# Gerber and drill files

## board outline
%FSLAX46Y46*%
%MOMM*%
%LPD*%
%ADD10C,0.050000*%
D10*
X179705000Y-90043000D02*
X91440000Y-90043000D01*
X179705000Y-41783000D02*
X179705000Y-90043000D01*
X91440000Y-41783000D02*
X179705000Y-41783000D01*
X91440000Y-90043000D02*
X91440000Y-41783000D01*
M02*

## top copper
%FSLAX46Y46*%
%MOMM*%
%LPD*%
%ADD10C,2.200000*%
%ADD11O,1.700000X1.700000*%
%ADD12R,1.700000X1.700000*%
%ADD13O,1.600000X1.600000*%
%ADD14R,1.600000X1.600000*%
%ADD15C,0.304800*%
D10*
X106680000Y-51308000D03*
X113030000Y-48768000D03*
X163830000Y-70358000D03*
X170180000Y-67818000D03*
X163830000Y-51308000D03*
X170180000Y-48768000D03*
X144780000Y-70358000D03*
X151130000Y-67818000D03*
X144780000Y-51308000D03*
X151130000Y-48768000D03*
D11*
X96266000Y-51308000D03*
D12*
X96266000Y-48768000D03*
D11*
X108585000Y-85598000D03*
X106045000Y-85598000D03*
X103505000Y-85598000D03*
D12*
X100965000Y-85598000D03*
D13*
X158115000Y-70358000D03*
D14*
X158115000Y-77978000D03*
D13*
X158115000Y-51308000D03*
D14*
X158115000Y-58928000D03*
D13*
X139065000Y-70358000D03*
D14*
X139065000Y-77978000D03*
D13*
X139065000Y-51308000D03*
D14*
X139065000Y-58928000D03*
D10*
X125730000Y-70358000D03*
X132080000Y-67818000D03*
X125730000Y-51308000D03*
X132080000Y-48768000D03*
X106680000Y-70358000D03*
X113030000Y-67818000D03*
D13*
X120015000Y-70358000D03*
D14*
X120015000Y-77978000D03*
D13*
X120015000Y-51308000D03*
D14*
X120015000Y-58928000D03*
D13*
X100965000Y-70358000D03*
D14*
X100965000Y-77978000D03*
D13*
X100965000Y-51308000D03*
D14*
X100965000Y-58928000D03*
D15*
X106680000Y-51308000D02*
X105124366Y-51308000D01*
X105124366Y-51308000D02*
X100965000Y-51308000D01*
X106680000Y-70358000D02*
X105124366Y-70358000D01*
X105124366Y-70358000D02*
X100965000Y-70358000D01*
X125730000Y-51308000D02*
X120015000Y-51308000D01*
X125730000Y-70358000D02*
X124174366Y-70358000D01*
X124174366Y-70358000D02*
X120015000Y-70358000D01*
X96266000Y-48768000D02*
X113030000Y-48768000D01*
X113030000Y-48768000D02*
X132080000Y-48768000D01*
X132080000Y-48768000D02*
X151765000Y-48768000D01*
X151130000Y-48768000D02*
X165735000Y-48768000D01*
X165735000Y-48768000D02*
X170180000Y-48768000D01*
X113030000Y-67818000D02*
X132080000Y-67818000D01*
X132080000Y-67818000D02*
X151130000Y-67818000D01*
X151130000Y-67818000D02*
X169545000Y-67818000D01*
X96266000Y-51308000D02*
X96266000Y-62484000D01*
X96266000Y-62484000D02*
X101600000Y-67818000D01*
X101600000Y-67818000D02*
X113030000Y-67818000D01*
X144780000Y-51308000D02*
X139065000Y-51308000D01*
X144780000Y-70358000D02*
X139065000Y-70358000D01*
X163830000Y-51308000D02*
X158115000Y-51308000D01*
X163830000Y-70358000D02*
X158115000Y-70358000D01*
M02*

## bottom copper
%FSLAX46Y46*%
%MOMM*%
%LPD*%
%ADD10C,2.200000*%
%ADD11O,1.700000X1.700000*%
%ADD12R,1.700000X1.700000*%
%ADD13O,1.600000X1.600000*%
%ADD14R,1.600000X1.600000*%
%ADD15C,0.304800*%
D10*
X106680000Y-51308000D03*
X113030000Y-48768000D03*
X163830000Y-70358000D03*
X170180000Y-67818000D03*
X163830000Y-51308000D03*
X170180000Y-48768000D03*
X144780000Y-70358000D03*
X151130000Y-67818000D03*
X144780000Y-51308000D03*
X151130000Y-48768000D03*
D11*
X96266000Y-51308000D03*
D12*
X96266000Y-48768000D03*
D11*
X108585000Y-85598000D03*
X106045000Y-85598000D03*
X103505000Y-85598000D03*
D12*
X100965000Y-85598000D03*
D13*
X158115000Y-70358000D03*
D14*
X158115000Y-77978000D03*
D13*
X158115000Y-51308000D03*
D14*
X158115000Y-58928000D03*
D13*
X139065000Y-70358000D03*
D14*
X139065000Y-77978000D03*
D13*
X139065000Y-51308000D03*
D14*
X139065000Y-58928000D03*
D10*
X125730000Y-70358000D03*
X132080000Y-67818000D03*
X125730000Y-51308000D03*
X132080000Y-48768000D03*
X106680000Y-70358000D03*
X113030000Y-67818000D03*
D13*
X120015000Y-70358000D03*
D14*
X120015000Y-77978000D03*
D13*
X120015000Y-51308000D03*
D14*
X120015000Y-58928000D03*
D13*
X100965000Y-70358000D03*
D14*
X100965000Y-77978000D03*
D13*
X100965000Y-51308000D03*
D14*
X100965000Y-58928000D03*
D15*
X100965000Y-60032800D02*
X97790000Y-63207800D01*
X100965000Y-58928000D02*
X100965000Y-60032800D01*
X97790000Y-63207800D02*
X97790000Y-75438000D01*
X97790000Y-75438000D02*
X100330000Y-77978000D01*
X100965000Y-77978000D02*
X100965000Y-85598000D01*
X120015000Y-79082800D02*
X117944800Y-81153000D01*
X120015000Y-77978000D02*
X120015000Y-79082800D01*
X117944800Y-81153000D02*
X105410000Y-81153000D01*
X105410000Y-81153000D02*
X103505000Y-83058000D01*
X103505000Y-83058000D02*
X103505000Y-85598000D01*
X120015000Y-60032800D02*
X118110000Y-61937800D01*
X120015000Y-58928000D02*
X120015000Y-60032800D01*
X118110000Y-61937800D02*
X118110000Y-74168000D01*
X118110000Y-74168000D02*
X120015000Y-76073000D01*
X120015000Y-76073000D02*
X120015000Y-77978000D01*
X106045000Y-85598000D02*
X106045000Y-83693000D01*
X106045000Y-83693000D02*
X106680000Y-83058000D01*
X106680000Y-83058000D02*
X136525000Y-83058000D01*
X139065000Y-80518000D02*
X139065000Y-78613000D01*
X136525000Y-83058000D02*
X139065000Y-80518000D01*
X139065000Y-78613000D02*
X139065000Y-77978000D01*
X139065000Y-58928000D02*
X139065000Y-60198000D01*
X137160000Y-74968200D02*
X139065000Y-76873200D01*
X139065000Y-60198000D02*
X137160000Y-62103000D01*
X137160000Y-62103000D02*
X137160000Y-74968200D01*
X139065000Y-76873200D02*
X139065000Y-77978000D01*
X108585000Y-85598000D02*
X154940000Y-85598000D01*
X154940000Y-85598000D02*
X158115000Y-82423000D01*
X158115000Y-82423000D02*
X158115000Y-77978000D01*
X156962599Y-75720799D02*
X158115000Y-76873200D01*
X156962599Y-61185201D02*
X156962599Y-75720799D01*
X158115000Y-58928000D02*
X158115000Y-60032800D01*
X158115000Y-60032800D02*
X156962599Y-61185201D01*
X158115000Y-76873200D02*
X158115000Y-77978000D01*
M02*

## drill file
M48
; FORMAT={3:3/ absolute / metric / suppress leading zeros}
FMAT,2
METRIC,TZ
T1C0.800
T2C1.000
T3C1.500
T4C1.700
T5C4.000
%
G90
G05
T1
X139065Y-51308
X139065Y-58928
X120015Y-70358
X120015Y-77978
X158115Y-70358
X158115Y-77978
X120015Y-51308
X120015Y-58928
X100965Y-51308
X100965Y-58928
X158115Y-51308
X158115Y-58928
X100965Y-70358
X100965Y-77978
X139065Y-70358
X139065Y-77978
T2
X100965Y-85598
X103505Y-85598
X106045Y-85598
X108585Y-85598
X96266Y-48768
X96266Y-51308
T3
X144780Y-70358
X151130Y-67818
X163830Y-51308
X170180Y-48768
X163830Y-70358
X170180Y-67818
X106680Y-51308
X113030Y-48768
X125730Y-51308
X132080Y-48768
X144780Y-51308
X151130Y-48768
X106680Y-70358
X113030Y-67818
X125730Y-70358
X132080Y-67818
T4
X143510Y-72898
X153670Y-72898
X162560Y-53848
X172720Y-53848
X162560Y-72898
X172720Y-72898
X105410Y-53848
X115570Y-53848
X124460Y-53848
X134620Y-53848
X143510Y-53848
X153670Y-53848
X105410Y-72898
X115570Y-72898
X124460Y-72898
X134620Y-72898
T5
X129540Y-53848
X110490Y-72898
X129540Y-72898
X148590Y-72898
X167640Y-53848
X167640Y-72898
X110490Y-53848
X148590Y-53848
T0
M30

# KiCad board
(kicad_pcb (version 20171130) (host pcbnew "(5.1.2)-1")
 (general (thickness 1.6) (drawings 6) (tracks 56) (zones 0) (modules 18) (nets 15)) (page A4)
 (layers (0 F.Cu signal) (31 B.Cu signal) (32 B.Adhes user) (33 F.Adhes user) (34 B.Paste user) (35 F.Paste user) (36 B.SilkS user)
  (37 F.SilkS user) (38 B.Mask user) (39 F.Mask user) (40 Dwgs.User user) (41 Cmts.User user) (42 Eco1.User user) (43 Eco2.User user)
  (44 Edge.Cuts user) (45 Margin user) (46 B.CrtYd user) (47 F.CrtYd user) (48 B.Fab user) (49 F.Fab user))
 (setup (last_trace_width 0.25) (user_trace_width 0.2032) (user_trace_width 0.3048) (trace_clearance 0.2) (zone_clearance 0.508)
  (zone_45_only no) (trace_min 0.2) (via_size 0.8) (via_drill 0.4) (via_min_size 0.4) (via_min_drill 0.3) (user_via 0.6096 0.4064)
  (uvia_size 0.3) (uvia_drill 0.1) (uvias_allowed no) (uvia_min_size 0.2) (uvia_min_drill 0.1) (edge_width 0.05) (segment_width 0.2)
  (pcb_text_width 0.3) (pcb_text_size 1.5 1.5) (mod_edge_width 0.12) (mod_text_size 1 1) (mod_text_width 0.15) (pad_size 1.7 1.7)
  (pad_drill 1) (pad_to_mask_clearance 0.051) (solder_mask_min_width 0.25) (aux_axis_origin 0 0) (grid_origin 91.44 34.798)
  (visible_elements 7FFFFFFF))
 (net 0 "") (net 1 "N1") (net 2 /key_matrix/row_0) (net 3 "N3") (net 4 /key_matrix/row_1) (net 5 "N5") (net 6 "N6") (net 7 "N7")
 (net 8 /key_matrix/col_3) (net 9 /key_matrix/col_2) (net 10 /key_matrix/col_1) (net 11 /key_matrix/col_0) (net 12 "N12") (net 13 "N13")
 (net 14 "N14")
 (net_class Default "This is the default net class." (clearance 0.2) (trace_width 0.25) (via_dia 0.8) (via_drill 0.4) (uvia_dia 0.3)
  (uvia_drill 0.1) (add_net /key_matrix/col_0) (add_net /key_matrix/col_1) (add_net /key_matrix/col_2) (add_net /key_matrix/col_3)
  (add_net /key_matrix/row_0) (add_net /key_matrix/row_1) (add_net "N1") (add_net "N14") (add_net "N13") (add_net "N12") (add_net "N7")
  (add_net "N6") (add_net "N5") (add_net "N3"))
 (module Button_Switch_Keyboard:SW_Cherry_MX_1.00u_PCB (layer F.Cu) (at 113.03 48.768)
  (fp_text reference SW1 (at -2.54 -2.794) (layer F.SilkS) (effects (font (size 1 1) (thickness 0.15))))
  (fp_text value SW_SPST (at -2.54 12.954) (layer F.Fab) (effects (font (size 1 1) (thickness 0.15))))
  (pad "" np_thru_hole circle (at 2.54 5.08) (size 1.7 1.7) (drill 1.7) (layers *.Cu *.Mask))
  (pad "" np_thru_hole circle (at -7.62 5.08) (size 1.7 1.7) (drill 1.7) (layers *.Cu *.Mask))
  (pad "" np_thru_hole circle (at -2.54 5.08) (size 4 4) (drill 4) (layers *.Cu *.Mask))
  (pad 2 thru_hole circle (at -6.35 2.54) (size 2.2 2.2) (drill 1.5) (layers *.Cu *.Mask) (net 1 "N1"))
  (pad 1 thru_hole circle (at 0 0) (size 2.2 2.2) (drill 1.5) (layers *.Cu *.Mask) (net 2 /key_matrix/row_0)))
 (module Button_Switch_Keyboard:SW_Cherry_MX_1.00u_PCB (layer F.Cu) (at 170.18 67.818)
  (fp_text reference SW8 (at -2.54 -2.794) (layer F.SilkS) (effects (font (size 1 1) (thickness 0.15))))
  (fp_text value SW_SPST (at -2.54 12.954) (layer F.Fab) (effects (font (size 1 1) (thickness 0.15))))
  (pad "" np_thru_hole circle (at 2.54 5.08) (size 1.7 1.7) (drill 1.7) (layers *.Cu *.Mask))
  (pad "" np_thru_hole circle (at -7.62 5.08) (size 1.7 1.7) (drill 1.7) (layers *.Cu *.Mask))
  (pad "" np_thru_hole circle (at -2.54 5.08) (size 4 4) (drill 4) (layers *.Cu *.Mask))
  (pad 2 thru_hole circle (at -6.35 2.54) (size 2.2 2.2) (drill 1.5) (layers *.Cu *.Mask) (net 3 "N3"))
  (pad 1 thru_hole circle (at 0 0) (size 2.2 2.2) (drill 1.5) (layers *.Cu *.Mask) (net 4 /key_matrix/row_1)))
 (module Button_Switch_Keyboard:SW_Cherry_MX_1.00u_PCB (layer F.Cu) (at 170.18 48.768)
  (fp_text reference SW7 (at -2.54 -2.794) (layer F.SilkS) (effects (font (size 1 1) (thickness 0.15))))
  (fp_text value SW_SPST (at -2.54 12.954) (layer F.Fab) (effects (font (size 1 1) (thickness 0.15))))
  (pad "" np_thru_hole circle (at 2.54 5.08) (size 1.7 1.7) (drill 1.7) (layers *.Cu *.Mask))
  (pad "" np_thru_hole circle (at -7.62 5.08) (size 1.7 1.7) (drill 1.7) (layers *.Cu *.Mask))
  (pad "" np_thru_hole circle (at -2.54 5.08) (size 4 4) (drill 4) (layers *.Cu *.Mask))
  (pad 2 thru_hole circle (at -6.35 2.54) (size 2.2 2.2) (drill 1.5) (layers *.Cu *.Mask) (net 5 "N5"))
  (pad 1 thru_hole circle (at 0 0) (size 2.2 2.2) (drill 1.5) (layers *.Cu *.Mask) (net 2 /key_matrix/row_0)))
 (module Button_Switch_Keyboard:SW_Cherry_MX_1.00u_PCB (layer F.Cu) (at 151.13 67.818)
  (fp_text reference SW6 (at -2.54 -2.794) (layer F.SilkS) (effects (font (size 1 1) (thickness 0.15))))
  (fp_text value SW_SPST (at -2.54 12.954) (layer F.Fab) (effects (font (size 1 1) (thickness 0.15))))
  (pad "" np_thru_hole circle (at 2.54 5.08) (size 1.7 1.7) (drill 1.7) (layers *.Cu *.Mask))
  (pad "" np_thru_hole circle (at -7.62 5.08) (size 1.7 1.7) (drill 1.7) (layers *.Cu *.Mask))
  (pad "" np_thru_hole circle (at -2.54 5.08) (size 4 4) (drill 4) (layers *.Cu *.Mask))
  (pad 2 thru_hole circle (at -6.35 2.54) (size 2.2 2.2) (drill 1.5) (layers *.Cu *.Mask) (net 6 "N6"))
  (pad 1 thru_hole circle (at 0 0) (size 2.2 2.2) (drill 1.5) (layers *.Cu *.Mask) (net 4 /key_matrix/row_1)))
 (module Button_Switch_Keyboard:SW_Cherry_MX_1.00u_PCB (layer F.Cu) (at 151.13 48.768)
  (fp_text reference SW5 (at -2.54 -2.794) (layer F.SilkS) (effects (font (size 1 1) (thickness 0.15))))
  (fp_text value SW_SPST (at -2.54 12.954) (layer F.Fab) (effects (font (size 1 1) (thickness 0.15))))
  (pad "" np_thru_hole circle (at 2.54 5.08) (size 1.7 1.7) (drill 1.7) (layers *.Cu *.Mask))
  (pad "" np_thru_hole circle (at -7.62 5.08) (size 1.7 1.7) (drill 1.7) (layers *.Cu *.Mask))
  (pad "" np_thru_hole circle (at -2.54 5.08) (size 4 4) (drill 4) (layers *.Cu *.Mask))
  (pad 2 thru_hole circle (at -6.35 2.54) (size 2.2 2.2) (drill 1.5) (layers *.Cu *.Mask) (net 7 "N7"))
  (pad 1 thru_hole circle (at 0 0) (size 2.2 2.2) (drill 1.5) (layers *.Cu *.Mask) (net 2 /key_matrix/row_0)))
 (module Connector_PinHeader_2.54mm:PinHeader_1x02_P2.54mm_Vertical (layer F.Cu) (at 96.266 48.768)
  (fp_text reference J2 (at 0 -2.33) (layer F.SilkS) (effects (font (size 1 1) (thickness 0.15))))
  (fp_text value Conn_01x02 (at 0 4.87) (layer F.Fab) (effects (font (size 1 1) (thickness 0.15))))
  (pad 2 thru_hole oval (at 0 2.54) (size 1.7 1.7) (drill 1) (layers *.Cu *.Mask) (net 4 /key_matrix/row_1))
  (pad 1 thru_hole rect (at 0 0) (size 1.7 1.7) (drill 1) (layers *.Cu *.Mask) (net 2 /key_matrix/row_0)))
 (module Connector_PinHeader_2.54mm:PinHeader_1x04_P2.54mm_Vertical (layer F.Cu) (at 100.965 85.598 90)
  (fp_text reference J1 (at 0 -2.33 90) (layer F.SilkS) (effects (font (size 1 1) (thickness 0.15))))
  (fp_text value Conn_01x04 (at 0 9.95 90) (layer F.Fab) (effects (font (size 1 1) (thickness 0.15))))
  (pad 4 thru_hole oval (at 0 7.62 90) (size 1.7 1.7) (drill 1) (layers *.Cu *.Mask) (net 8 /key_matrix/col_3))
  (pad 3 thru_hole oval (at 0 5.08 90) (size 1.7 1.7) (drill 1) (layers *.Cu *.Mask) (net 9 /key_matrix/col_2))
  (pad 2 thru_hole oval (at 0 2.54 90) (size 1.7 1.7) (drill 1) (layers *.Cu *.Mask) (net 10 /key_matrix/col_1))
  (pad 1 thru_hole rect (at 0 0 90) (size 1.7 1.7) (drill 1) (layers *.Cu *.Mask) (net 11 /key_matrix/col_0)))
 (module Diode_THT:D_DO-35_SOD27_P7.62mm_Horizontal (layer F.Cu) (at 158.115 77.978 90)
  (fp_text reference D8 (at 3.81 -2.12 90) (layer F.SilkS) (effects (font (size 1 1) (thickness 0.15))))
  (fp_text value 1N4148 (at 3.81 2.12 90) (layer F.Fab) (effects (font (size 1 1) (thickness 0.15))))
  (pad 2 thru_hole oval (at 7.62 0 90) (size 1.6 1.6) (drill 0.8) (layers *.Cu *.Mask) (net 3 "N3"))
  (pad 1 thru_hole rect (at 0 0 90) (size 1.6 1.6) (drill 0.8) (layers *.Cu *.Mask) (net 8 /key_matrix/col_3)))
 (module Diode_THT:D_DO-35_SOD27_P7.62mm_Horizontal (layer F.Cu) (at 158.115 58.928 90)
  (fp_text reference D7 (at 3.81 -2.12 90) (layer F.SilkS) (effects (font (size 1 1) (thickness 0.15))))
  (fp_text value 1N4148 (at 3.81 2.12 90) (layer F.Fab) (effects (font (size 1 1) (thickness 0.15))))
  (pad 2 thru_hole oval (at 7.62 0 90) (size 1.6 1.6) (drill 0.8) (layers *.Cu *.Mask) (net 5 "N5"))
  (pad 1 thru_hole rect (at 0 0 90) (size 1.6 1.6) (drill 0.8) (layers *.Cu *.Mask) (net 8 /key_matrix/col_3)))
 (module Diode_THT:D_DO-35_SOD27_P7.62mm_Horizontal (layer F.Cu) (at 139.065 77.978 90)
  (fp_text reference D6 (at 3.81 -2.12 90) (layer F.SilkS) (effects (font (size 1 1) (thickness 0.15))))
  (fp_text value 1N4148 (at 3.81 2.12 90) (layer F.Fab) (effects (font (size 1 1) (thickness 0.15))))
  (pad 2 thru_hole oval (at 7.62 0 90) (size 1.6 1.6) (drill 0.8) (layers *.Cu *.Mask) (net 6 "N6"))
  (pad 1 thru_hole rect (at 0 0 90) (size 1.6 1.6) (drill 0.8) (layers *.Cu *.Mask) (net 9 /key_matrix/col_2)))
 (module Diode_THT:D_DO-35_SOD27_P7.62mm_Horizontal (layer F.Cu) (at 139.065 58.928 90)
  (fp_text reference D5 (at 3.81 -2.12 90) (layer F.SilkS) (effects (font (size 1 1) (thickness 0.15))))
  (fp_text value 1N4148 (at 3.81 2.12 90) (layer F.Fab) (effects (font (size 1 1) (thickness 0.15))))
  (pad 2 thru_hole oval (at 7.62 0 90) (size 1.6 1.6) (drill 0.8) (layers *.Cu *.Mask) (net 7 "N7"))
  (pad 1 thru_hole rect (at 0 0 90) (size 1.6 1.6) (drill 0.8) (layers *.Cu *.Mask) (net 9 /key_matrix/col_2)))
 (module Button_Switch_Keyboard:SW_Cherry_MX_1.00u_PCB (layer F.Cu) (at 132.08 67.818)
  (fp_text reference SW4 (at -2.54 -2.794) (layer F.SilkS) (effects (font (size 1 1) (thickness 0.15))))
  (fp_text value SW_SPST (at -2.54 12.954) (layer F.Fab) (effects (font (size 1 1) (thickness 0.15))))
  (pad "" np_thru_hole circle (at 2.54 5.08) (size 1.7 1.7) (drill 1.7) (layers *.Cu *.Mask))
  (pad "" np_thru_hole circle (at -7.62 5.08) (size 1.7 1.7) (drill 1.7) (layers *.Cu *.Mask))
  (pad "" np_thru_hole circle (at -2.54 5.08) (size 4 4) (drill 4) (layers *.Cu *.Mask))
  (pad 2 thru_hole circle (at -6.35 2.54) (size 2.2 2.2) (drill 1.5) (layers *.Cu *.Mask) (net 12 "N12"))
  (pad 1 thru_hole circle (at 0 0) (size 2.2 2.2) (drill 1.5) (layers *.Cu *.Mask) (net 4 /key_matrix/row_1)))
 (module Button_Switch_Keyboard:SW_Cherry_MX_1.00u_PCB (layer F.Cu) (at 132.08 48.768)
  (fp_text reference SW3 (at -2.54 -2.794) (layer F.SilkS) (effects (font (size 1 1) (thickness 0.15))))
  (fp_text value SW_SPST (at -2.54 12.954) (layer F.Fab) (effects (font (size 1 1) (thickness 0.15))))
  (pad "" np_thru_hole circle (at 2.54 5.08) (size 1.7 1.7) (drill 1.7) (layers *.Cu *.Mask))
  (pad "" np_thru_hole circle (at -7.62 5.08) (size 1.7 1.7) (drill 1.7) (layers *.Cu *.Mask))
  (pad "" np_thru_hole circle (at -2.54 5.08) (size 4 4) (drill 4) (layers *.Cu *.Mask))
  (pad 2 thru_hole circle (at -6.35 2.54) (size 2.2 2.2) (drill 1.5) (layers *.Cu *.Mask) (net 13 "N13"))
  (pad 1 thru_hole circle (at 0 0) (size 2.2 2.2) (drill 1.5) (layers *.Cu *.Mask) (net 2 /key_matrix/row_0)))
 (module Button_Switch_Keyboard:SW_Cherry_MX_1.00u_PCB (layer F.Cu) (at 113.03 67.818)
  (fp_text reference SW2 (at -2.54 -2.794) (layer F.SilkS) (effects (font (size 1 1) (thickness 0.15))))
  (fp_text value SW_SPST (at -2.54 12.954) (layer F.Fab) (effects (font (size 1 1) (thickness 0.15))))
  (pad "" np_thru_hole circle (at 2.54 5.08) (size 1.7 1.7) (drill 1.7) (layers *.Cu *.Mask))
  (pad "" np_thru_hole circle (at -7.62 5.08) (size 1.7 1.7) (drill 1.7) (layers *.Cu *.Mask))
  (pad "" np_thru_hole circle (at -2.54 5.08) (size 4 4) (drill 4) (layers *.Cu *.Mask))
  (pad 2 thru_hole circle (at -6.35 2.54) (size 2.2 2.2) (drill 1.5) (layers *.Cu *.Mask) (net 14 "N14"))
  (pad 1 thru_hole circle (at 0 0) (size 2.2 2.2) (drill 1.5) (layers *.Cu *.Mask) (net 4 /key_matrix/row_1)))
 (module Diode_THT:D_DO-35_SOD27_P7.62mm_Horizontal (layer F.Cu) (at 120.015 77.978 90)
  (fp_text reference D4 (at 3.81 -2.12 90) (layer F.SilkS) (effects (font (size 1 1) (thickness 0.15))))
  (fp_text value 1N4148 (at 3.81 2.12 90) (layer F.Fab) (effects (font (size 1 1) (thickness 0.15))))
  (pad 2 thru_hole oval (at 7.62 0 90) (size 1.6 1.6) (drill 0.8) (layers *.Cu *.Mask) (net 12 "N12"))
  (pad 1 thru_hole rect (at 0 0 90) (size 1.6 1.6) (drill 0.8) (layers *.Cu *.Mask) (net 10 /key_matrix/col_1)))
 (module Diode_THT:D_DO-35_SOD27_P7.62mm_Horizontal (layer F.Cu) (at 120.015 58.928 90)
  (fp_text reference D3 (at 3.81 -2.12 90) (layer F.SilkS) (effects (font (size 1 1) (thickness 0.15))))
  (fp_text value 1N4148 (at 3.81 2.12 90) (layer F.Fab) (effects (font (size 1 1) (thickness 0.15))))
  (pad 2 thru_hole oval (at 7.62 0 90) (size 1.6 1.6) (drill 0.8) (layers *.Cu *.Mask) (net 13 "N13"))
  (pad 1 thru_hole rect (at 0 0 90) (size 1.6 1.6) (drill 0.8) (layers *.Cu *.Mask) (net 10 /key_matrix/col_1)))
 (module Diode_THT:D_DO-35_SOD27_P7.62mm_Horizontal (layer F.Cu) (at 100.965 77.978 90)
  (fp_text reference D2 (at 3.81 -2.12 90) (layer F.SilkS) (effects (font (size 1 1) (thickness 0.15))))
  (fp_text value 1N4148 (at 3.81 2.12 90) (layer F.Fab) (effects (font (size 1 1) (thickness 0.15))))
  (pad 2 thru_hole oval (at 7.62 0 90) (size 1.6 1.6) (drill 0.8) (layers *.Cu *.Mask) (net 14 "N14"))
  (pad 1 thru_hole rect (at 0 0 90) (size 1.6 1.6) (drill 0.8) (layers *.Cu *.Mask) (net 11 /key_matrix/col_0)))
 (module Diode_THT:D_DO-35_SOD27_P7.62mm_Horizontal (layer F.Cu) (at 100.965 58.928 90)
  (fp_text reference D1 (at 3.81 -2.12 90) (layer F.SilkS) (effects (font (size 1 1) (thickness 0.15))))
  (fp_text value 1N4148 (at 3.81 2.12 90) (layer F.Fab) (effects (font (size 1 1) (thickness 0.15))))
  (pad 2 thru_hole oval (at 7.62 0 90) (size 1.6 1.6) (drill 0.8) (layers *.Cu *.Mask) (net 1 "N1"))
  (pad 1 thru_hole rect (at 0 0 90) (size 1.6 1.6) (drill 0.8) (layers *.Cu *.Mask) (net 11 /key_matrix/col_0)))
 (gr_line (start 179.705 90.043) (end 91.44 90.043) (layer Edge.Cuts) (width 0.05))
 (gr_line (start 179.705 41.783) (end 179.705 90.043) (layer Edge.Cuts) (width 0.05))
 (gr_line (start 91.44 41.783) (end 179.705 41.783) (layer Edge.Cuts) (width 0.05))
 (gr_line (start 91.44 90.043) (end 91.44 41.783) (layer Edge.Cuts) (width 0.05))
 (segment (start 106.68 51.308) (end 105.124366 51.308) (width 0.3048) (layer F.Cu) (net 1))
 (segment (start 105.124366 51.308) (end 100.965 51.308) (width 0.3048) (layer F.Cu) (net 1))
 (segment (start 100.965 60.0328) (end 97.79 63.2078) (width 0.3048) (layer B.Cu) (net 11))
 (segment (start 100.965 58.928) (end 100.965 60.0328) (width 0.3048) (layer B.Cu) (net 11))
 (segment (start 97.79 63.2078) (end 97.79 75.438) (width 0.3048) (layer B.Cu) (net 11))
 (segment (start 97.79 75.438) (end 100.33 77.978) (width 0.3048) (layer B.Cu) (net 11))
 (segment (start 100.965 77.978) (end 100.965 85.598) (width 0.3048) (layer B.Cu) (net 11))
 (segment (start 106.68 70.358) (end 105.124366 70.358) (width 0.3048) (layer F.Cu) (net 14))
 (segment (start 105.124366 70.358) (end 100.965 70.358) (width 0.3048) (layer F.Cu) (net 14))
 (segment (start 125.73 51.308) (end 120.015 51.308) (width 0.3048) (layer F.Cu) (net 13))
 (segment (start 120.015 79.0828) (end 117.9448 81.153) (width 0.3048) (layer B.Cu) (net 10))
 (segment (start 120.015 77.978) (end 120.015 79.0828) (width 0.3048) (layer B.Cu) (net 10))
 (segment (start 117.9448 81.153) (end 105.41 81.153) (width 0.3048) (layer B.Cu) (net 10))
 (segment (start 105.41 81.153) (end 103.505 83.058) (width 0.3048) (layer B.Cu) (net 10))
 (segment (start 103.505 83.058) (end 103.505 85.598) (width 0.3048) (layer B.Cu) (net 10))
 (segment (start 120.015 60.0328) (end 118.11 61.9378) (width 0.3048) (layer B.Cu) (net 10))
 (segment (start 120.015 58.928) (end 120.015 60.0328) (width 0.3048) (layer B.Cu) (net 10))
 (segment (start 118.11 61.9378) (end 118.11 74.168) (width 0.3048) (layer B.Cu) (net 10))
 (segment (start 118.11 74.168) (end 120.015 76.073) (width 0.3048) (layer B.Cu) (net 10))
 (segment (start 120.015 76.073) (end 120.015 77.978) (width 0.3048) (layer B.Cu) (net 10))
 (segment (start 125.73 70.358) (end 124.174366 70.358) (width 0.3048) (layer F.Cu) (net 12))
 (segment (start 124.174366 70.358) (end 120.015 70.358) (width 0.3048) (layer F.Cu) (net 12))
 (segment (start 96.266 48.768) (end 113.03 48.768) (width 0.3048) (layer F.Cu) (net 2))
 (segment (start 113.03 48.768) (end 132.08 48.768) (width 0.3048) (layer F.Cu) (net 2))
 (segment (start 132.08 48.768) (end 151.765 48.768) (width 0.3048) (layer F.Cu) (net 2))
 (segment (start 151.13 48.768) (end 165.735 48.768) (width 0.3048) (layer F.Cu) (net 2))
 (segment (start 165.735 48.768) (end 170.18 48.768) (width 0.3048) (layer F.Cu) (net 2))
 (segment (start 113.03 67.818) (end 132.08 67.818) (width 0.3048) (layer F.Cu) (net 4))
 (segment (start 132.08 67.818) (end 151.13 67.818) (width 0.3048) (layer F.Cu) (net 4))
 (segment (start 151.13 67.818) (end 169.545 67.818) (width 0.3048) (layer F.Cu) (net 4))
 (segment (start 96.266 51.308) (end 96.266 62.484) (width 0.3048) (layer F.Cu) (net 4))
 (segment (start 96.266 62.484) (end 101.6 67.818) (width 0.3048) (layer F.Cu) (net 4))
 (segment (start 101.6 67.818) (end 113.03 67.818) (width 0.3048) (layer F.Cu) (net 4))
 (segment (start 144.78 51.308) (end 139.065 51.308) (width 0.3048) (layer F.Cu) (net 7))
 (segment (start 106.045 85.598) (end 106.045 83.693) (width 0.3048) (layer B.Cu) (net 9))
 (segment (start 106.045 83.693) (end 106.68 83.058) (width 0.3048) (layer B.Cu) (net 9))
 (segment (start 106.68 83.058) (end 136.525 83.058) (width 0.3048) (layer B.Cu) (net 9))
 (segment (start 139.065 80.518) (end 139.065 78.613) (width 0.3048) (layer B.Cu) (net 9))
 (segment (start 136.525 83.058) (end 139.065 80.518) (width 0.3048) (layer B.Cu) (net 9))
 (segment (start 139.065 78.613) (end 139.065 77.978) (width 0.3048) (layer B.Cu) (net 9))
 (segment (start 139.065 58.928) (end 139.065 60.198) (width 0.3048) (layer B.Cu) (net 9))
 (segment (start 137.16 74.9682) (end 139.065 76.8732) (width 0.3048) (layer B.Cu) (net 9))
 (segment (start 139.065 60.198) (end 137.16 62.103) (width 0.3048) (layer B.Cu) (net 9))
 (segment (start 137.16 62.103) (end 137.16 74.9682) (width 0.3048) (layer B.Cu) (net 9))
 (segment (start 139.065 76.8732) (end 139.065 77.978) (width 0.3048) (layer B.Cu) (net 9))
 (segment (start 144.78 70.358) (end 139.065 70.358) (width 0.3048) (layer F.Cu) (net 6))
 (segment (start 163.83 51.308) (end 158.115 51.308) (width 0.3048) (layer F.Cu) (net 5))
 (segment (start 108.585 85.598) (end 154.94 85.598) (width 0.3048) (layer B.Cu) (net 8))
 (segment (start 154.94 85.598) (end 158.115 82.423) (width 0.3048) (layer B.Cu) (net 8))
 (segment (start 158.115 82.423) (end 158.115 77.978) (width 0.3048) (layer B.Cu) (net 8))
 (segment (start 156.962599 75.720799) (end 158.115 76.8732) (width 0.3048) (layer B.Cu) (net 8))
 (segment (start 156.962599 61.185201) (end 156.962599 75.720799) (width 0.3048) (layer B.Cu) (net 8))
 (segment (start 158.115 58.928) (end 158.115 60.0328) (width 0.3048) (layer B.Cu) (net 8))
 (segment (start 158.115 60.0328) (end 156.962599 61.185201) (width 0.3048) (layer B.Cu) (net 8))
 (segment (start 158.115 76.8732) (end 158.115 77.978) (width 0.3048) (layer B.Cu) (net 8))
 (segment (start 163.83 70.358) (end 158.115 70.358) (width 0.3048) (layer F.Cu) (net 3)))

